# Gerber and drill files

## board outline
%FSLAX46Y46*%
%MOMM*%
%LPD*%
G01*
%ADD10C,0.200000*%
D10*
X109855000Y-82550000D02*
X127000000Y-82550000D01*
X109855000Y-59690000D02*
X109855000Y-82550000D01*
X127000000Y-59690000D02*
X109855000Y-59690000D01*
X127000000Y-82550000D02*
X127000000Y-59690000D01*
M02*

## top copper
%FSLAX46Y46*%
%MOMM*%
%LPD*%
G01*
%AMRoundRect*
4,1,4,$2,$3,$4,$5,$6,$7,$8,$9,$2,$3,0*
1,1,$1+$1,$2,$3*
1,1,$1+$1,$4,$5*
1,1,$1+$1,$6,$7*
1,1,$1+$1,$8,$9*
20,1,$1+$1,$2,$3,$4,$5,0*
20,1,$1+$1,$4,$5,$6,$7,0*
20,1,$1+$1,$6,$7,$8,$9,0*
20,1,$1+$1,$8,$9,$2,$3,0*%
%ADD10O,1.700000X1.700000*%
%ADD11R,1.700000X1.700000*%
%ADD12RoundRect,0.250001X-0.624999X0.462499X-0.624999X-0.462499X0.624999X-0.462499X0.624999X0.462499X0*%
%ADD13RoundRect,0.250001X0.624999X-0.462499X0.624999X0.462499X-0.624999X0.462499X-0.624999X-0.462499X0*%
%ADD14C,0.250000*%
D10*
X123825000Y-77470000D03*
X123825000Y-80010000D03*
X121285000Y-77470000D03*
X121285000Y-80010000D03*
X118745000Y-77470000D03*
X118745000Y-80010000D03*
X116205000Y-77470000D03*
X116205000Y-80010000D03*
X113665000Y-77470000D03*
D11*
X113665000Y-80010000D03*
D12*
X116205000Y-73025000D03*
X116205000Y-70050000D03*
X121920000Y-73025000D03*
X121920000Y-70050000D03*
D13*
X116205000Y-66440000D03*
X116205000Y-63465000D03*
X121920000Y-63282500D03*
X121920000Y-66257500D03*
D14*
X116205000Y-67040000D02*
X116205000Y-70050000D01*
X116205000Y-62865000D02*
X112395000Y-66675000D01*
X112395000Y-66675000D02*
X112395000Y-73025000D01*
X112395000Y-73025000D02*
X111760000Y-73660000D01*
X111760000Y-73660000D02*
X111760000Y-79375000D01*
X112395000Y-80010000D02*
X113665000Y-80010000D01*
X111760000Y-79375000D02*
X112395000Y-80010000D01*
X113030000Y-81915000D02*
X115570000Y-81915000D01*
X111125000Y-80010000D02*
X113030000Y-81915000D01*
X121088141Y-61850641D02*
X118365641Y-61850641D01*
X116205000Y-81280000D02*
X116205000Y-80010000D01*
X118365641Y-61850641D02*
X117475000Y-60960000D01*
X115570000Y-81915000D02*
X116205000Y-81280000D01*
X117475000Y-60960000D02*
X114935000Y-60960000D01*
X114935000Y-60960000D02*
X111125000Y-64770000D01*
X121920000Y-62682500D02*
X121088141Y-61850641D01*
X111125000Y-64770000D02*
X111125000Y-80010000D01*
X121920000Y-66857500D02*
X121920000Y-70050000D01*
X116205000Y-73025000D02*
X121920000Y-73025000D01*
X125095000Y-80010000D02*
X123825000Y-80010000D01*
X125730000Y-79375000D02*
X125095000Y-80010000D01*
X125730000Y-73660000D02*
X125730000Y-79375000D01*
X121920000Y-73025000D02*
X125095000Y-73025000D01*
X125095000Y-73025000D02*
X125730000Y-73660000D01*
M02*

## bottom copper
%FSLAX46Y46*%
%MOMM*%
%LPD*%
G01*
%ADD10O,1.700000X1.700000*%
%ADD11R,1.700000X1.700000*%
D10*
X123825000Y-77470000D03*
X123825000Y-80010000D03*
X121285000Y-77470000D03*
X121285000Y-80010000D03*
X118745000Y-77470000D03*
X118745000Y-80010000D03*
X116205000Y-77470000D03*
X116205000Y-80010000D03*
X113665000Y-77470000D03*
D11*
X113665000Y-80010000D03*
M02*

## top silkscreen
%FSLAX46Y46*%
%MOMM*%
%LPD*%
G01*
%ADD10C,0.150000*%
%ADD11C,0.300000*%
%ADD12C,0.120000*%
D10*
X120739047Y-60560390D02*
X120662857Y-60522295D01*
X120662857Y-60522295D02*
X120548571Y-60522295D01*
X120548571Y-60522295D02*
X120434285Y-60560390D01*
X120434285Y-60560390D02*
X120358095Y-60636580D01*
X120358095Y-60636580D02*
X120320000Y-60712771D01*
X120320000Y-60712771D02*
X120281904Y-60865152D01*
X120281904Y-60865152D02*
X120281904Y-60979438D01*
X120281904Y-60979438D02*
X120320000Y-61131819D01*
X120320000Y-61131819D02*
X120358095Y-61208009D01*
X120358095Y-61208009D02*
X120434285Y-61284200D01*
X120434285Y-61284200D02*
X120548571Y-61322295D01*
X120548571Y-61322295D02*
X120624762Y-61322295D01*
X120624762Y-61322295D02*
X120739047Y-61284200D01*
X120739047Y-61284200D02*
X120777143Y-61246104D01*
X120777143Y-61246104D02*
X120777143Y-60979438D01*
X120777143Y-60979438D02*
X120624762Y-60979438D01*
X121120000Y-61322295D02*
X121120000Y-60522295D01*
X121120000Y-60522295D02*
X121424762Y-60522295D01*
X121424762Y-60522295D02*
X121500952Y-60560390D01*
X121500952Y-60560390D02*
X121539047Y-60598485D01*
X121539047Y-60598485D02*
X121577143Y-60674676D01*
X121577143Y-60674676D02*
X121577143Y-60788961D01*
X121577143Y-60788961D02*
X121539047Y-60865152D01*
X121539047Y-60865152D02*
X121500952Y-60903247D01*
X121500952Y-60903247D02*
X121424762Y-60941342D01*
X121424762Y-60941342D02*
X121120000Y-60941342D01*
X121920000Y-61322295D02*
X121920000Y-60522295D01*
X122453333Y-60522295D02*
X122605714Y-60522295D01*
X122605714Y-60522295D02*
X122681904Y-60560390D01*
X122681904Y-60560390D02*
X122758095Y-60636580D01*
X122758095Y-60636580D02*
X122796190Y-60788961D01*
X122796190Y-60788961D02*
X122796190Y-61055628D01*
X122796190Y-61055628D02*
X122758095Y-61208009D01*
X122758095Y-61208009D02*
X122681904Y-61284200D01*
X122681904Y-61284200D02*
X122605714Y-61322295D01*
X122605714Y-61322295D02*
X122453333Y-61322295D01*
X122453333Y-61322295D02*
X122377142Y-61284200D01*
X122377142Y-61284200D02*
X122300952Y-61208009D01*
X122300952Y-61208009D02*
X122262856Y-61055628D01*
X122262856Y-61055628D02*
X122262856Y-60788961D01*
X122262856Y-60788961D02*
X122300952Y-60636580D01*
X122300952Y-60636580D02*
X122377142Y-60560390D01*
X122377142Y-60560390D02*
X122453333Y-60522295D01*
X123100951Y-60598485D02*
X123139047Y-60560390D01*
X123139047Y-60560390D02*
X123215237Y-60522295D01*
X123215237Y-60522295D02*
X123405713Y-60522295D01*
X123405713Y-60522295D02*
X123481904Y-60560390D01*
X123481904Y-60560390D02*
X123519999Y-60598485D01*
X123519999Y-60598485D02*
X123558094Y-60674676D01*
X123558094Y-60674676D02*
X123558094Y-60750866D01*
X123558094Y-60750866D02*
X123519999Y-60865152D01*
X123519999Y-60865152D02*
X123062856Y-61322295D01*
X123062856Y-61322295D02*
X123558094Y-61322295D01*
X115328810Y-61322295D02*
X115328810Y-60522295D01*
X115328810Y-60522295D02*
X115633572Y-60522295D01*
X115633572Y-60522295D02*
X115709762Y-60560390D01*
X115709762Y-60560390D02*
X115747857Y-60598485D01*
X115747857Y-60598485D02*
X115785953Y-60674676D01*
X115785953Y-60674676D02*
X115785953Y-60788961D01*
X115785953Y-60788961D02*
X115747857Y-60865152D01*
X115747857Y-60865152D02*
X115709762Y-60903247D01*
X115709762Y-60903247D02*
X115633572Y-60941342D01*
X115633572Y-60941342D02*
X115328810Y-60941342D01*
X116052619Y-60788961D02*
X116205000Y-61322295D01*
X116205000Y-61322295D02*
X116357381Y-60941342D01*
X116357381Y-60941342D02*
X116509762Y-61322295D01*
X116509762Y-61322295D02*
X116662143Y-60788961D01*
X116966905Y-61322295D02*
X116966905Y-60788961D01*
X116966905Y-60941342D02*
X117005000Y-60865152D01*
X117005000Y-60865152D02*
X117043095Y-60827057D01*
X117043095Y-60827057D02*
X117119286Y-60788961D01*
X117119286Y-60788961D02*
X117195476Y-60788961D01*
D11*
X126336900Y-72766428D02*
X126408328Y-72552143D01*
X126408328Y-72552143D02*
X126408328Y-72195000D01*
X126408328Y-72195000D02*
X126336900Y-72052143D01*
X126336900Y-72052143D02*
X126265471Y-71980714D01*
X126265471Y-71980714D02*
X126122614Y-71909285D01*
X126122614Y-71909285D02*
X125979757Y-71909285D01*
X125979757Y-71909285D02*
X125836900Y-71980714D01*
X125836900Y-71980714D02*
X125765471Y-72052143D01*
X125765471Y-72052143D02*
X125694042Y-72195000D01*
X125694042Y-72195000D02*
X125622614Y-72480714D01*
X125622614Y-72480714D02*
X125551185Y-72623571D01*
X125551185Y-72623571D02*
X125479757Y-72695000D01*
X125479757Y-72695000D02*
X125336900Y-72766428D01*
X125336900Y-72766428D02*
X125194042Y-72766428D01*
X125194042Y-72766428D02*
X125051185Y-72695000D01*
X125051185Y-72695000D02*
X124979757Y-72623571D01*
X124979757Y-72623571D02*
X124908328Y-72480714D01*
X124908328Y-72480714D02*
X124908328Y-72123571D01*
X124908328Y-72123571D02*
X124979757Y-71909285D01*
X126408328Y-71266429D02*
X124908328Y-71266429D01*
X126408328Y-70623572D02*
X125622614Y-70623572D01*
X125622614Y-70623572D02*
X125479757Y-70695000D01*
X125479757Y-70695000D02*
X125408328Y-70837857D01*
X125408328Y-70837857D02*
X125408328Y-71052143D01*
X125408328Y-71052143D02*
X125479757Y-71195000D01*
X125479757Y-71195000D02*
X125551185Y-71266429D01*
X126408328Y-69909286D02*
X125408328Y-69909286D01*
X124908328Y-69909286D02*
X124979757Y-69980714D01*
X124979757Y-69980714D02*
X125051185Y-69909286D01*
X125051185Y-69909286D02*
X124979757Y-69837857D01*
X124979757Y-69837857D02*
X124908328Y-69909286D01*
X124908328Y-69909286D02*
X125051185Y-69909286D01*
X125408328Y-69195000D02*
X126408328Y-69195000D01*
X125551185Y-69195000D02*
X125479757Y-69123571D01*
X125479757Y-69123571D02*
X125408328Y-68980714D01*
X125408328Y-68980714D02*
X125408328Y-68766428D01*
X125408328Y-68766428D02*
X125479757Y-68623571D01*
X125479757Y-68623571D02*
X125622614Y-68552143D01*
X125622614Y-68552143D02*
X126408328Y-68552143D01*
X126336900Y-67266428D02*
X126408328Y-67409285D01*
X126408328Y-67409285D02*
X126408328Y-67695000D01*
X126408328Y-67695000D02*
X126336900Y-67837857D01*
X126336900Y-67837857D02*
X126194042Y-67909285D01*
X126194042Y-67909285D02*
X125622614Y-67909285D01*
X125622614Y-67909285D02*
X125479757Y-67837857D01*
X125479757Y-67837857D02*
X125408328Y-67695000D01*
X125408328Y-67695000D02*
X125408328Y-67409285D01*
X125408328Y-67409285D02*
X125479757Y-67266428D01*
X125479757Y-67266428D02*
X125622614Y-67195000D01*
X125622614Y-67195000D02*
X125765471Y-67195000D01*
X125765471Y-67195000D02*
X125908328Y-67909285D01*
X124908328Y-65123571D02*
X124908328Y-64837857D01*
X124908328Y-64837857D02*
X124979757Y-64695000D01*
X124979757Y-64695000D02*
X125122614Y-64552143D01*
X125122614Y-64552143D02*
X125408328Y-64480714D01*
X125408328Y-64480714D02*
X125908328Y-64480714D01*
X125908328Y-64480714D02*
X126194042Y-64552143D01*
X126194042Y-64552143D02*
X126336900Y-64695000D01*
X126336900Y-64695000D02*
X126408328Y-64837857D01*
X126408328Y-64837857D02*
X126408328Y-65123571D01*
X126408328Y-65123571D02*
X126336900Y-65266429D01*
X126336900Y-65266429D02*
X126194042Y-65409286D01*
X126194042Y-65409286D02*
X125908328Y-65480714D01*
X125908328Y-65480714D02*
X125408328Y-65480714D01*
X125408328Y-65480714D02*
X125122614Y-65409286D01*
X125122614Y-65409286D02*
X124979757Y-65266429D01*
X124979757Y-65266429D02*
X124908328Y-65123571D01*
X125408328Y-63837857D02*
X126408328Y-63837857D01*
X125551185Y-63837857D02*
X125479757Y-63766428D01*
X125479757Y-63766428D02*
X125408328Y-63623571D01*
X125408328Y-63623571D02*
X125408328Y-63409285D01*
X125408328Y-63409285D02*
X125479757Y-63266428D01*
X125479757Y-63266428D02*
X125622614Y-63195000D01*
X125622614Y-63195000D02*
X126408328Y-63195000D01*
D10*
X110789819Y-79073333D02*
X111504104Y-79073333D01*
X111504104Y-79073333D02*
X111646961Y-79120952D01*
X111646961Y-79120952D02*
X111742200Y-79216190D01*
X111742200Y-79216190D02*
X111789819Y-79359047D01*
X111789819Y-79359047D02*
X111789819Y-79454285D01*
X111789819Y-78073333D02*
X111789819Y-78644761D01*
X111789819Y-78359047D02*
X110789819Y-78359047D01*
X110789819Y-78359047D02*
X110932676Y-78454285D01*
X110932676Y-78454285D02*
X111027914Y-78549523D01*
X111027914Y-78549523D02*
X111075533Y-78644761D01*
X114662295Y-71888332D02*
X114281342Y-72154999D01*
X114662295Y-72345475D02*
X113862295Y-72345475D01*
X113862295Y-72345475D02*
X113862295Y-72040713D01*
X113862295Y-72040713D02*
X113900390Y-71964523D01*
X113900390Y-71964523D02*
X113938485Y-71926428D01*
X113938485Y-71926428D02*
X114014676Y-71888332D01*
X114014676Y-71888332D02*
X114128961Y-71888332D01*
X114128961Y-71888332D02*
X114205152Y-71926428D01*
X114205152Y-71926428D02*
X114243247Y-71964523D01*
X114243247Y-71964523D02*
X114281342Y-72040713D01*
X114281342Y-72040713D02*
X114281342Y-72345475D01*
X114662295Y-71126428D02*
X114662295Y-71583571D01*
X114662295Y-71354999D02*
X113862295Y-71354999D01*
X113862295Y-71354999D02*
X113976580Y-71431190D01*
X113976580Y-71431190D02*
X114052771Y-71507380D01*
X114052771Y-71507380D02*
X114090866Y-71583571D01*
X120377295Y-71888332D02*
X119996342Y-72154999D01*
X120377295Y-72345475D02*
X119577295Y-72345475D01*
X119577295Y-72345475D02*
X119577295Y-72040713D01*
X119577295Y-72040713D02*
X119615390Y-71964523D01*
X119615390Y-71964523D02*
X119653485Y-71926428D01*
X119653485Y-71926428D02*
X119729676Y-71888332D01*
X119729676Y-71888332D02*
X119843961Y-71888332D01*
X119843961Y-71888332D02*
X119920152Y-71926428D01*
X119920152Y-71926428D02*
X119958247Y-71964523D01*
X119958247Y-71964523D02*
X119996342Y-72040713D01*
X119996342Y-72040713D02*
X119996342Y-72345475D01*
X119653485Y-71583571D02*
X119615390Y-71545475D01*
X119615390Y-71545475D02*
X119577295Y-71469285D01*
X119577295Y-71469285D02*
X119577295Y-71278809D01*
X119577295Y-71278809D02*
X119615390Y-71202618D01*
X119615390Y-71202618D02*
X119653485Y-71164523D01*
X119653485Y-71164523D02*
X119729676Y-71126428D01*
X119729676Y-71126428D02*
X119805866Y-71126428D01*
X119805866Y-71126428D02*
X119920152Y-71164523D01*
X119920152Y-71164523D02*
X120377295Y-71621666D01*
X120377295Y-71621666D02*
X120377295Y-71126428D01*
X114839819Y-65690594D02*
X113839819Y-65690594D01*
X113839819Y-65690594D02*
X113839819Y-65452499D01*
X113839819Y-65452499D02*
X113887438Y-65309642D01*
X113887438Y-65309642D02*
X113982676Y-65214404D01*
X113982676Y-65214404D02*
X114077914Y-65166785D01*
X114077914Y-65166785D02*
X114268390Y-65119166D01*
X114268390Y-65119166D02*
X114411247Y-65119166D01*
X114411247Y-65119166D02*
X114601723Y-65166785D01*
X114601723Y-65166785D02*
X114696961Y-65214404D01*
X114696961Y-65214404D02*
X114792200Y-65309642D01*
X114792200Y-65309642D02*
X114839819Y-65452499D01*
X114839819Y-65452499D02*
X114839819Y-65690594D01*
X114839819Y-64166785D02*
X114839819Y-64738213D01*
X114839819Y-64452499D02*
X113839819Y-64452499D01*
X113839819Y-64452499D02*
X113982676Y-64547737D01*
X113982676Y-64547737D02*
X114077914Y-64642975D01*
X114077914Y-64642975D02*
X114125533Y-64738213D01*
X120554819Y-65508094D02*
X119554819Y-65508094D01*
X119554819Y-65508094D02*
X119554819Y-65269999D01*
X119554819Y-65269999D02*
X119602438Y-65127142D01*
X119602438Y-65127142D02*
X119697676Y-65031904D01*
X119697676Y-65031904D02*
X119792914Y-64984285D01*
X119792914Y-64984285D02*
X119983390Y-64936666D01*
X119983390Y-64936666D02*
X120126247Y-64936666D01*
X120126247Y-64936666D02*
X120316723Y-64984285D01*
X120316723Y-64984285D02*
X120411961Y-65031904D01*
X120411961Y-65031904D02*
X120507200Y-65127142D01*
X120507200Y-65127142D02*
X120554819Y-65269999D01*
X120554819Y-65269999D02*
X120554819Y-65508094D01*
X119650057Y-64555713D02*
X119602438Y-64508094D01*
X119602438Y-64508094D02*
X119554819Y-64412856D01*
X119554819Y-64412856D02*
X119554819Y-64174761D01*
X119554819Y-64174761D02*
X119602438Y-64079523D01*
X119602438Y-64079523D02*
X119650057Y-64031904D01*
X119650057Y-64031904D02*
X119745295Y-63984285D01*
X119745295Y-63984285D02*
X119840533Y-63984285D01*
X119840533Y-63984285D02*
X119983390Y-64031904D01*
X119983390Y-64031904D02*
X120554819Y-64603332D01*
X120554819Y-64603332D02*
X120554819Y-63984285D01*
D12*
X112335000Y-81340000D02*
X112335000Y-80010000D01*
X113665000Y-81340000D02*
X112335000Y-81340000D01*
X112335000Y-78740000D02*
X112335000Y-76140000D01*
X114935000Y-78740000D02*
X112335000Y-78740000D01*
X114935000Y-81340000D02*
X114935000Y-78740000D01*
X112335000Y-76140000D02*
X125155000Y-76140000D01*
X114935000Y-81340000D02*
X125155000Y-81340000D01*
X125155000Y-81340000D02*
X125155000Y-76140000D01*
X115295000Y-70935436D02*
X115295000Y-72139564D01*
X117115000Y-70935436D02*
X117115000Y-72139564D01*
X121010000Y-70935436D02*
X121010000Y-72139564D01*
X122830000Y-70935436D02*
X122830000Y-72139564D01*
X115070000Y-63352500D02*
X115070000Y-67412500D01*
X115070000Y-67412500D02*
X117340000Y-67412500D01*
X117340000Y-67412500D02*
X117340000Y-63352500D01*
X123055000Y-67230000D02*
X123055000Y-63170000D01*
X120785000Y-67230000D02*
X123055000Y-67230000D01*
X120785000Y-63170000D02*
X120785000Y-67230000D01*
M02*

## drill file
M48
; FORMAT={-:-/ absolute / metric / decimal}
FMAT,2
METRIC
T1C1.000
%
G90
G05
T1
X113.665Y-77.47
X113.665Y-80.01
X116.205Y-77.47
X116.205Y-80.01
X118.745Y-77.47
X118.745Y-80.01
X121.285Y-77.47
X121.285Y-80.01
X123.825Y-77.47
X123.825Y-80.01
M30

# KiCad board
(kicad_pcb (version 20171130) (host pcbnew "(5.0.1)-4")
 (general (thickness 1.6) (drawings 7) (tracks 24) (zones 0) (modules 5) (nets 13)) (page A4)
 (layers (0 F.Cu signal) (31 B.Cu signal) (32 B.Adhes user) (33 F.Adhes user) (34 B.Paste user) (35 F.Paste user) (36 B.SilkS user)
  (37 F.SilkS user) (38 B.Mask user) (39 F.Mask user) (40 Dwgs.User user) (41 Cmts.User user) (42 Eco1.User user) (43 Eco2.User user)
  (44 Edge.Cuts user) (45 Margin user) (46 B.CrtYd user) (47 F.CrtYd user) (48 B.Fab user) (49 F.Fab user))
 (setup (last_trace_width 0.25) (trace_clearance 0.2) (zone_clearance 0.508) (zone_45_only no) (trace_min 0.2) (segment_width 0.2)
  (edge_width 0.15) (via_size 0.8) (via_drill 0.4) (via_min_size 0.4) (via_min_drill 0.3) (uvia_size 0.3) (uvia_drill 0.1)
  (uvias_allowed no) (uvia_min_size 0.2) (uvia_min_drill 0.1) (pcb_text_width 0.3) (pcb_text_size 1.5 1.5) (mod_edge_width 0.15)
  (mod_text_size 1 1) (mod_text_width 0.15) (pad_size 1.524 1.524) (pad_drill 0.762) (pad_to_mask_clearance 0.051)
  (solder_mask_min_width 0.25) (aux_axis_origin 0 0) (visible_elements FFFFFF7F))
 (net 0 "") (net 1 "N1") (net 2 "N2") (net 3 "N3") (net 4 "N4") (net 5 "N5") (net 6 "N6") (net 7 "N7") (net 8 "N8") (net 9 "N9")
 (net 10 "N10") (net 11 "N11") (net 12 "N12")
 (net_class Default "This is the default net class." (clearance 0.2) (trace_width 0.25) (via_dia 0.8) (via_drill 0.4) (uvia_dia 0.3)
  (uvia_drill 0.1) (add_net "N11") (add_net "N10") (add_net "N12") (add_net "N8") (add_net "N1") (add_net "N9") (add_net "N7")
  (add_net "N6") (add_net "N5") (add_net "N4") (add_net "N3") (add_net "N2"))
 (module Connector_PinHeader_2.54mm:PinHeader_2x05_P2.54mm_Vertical (layer F.Cu) (at 113.665 80.01 90)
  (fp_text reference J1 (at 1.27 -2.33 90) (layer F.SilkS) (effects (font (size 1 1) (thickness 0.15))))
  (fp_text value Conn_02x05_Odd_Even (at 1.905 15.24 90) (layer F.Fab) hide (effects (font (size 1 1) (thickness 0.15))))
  (fp_line (start -1.33 -1.33) (end 0 -1.33) (layer F.SilkS) (width 0.12))
  (fp_line (start -1.33 0) (end -1.33 -1.33) (layer F.SilkS) (width 0.12))
  (fp_line (start 1.27 -1.33) (end 3.87 -1.33) (layer F.SilkS) (width 0.12))
  (fp_line (start 1.27 1.27) (end 1.27 -1.33) (layer F.SilkS) (width 0.12))
  (fp_line (start -1.33 1.27) (end 1.27 1.27) (layer F.SilkS) (width 0.12))
  (fp_line (start 3.87 -1.33) (end 3.87 11.49) (layer F.SilkS) (width 0.12))
  (fp_line (start -1.33 1.27) (end -1.33 11.49) (layer F.SilkS) (width 0.12))
  (fp_line (start -1.33 11.49) (end 3.87 11.49) (layer F.SilkS) (width 0.12))
  (pad 10 thru_hole oval (at 2.54 10.16 90) (size 1.7 1.7) (drill 1) (layers *.Cu *.Mask) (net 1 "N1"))
  (pad 9 thru_hole oval (at 0 10.16 90) (size 1.7 1.7) (drill 1) (layers *.Cu *.Mask) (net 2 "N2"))
  (pad 8 thru_hole oval (at 2.54 7.62 90) (size 1.7 1.7) (drill 1) (layers *.Cu *.Mask) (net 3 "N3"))
  (pad 7 thru_hole oval (at 0 7.62 90) (size 1.7 1.7) (drill 1) (layers *.Cu *.Mask) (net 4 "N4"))
  (pad 6 thru_hole oval (at 2.54 5.08 90) (size 1.7 1.7) (drill 1) (layers *.Cu *.Mask) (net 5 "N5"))
  (pad 5 thru_hole oval (at 0 5.08 90) (size 1.7 1.7) (drill 1) (layers *.Cu *.Mask) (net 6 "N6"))
  (pad 4 thru_hole oval (at 2.54 2.54 90) (size 1.7 1.7) (drill 1) (layers *.Cu *.Mask) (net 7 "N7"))
  (pad 3 thru_hole oval (at 0 2.54 90) (size 1.7 1.7) (drill 1) (layers *.Cu *.Mask) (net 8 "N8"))
  (pad 2 thru_hole oval (at 2.54 0 90) (size 1.7 1.7) (drill 1) (layers *.Cu *.Mask) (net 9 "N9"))
  (pad 1 thru_hole rect (at 0 0 90) (size 1.7 1.7) (drill 1) (layers *.Cu *.Mask) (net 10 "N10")))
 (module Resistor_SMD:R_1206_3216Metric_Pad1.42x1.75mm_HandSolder (layer F.Cu) (at 116.205 71.5375 270)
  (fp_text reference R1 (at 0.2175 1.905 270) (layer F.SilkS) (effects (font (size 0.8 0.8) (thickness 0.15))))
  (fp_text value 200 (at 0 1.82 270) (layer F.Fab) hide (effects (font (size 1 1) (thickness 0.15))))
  (fp_line (start -0.602064 0.91) (end 0.602064 0.91) (layer F.SilkS) (width 0.12))
  (fp_line (start -0.602064 -0.91) (end 0.602064 -0.91) (layer F.SilkS) (width 0.12))
  (pad 2 smd roundrect (at 1.4875 0 270) (size 1.425 1.75) (layers F.Cu F.Paste F.Mask) (roundrect_rratio 0.175439) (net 2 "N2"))
  (pad 1 smd roundrect (at -1.4875 0 270) (size 1.425 1.75) (layers F.Cu F.Paste F.Mask) (roundrect_rratio 0.175439) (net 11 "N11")))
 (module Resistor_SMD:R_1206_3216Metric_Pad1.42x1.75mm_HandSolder (layer F.Cu) (at 121.92 71.5375 270)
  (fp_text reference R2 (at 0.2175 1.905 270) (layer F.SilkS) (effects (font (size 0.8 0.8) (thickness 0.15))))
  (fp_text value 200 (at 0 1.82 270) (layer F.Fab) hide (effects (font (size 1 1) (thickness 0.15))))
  (fp_line (start -0.602064 0.91) (end 0.602064 0.91) (layer F.SilkS) (width 0.12))
  (fp_line (start -0.602064 -0.91) (end 0.602064 -0.91) (layer F.SilkS) (width 0.12))
  (pad 2 smd roundrect (at 1.4875 0 270) (size 1.425 1.75) (layers F.Cu F.Paste F.Mask) (roundrect_rratio 0.175439) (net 2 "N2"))
  (pad 1 smd roundrect (at -1.4875 0 270) (size 1.425 1.75) (layers F.Cu F.Paste F.Mask) (roundrect_rratio 0.175439) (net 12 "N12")))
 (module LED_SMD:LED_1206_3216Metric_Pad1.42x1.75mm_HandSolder (layer F.Cu) (at 116.205 64.9525 90)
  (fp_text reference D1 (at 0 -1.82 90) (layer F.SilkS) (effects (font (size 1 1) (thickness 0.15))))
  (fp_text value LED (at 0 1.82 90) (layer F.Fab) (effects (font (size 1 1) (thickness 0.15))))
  (fp_line (start 1.6 -1.135) (end -2.46 -1.135) (layer F.SilkS) (width 0.12))
  (fp_line (start -2.46 -1.135) (end -2.46 1.135) (layer F.SilkS) (width 0.12))
  (fp_line (start -2.46 1.135) (end 1.6 1.135) (layer F.SilkS) (width 0.12))
  (pad 1 smd roundrect (at -1.4875 0 90) (size 1.425 1.75) (layers F.Cu F.Paste F.Mask) (roundrect_rratio 0.175439) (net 11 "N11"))
  (pad 2 smd roundrect (at 1.4875 0 90) (size 1.425 1.75) (layers F.Cu F.Paste F.Mask) (roundrect_rratio 0.175439) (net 10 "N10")))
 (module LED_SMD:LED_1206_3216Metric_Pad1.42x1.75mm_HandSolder (layer F.Cu) (at 121.92 64.77 90)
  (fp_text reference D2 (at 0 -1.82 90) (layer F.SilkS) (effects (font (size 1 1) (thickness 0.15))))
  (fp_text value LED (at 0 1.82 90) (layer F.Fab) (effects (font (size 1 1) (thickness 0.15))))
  (fp_line (start -2.46 1.135) (end 1.6 1.135) (layer F.SilkS) (width 0.12))
  (fp_line (start -2.46 -1.135) (end -2.46 1.135) (layer F.SilkS) (width 0.12))
  (fp_line (start 1.6 -1.135) (end -2.46 -1.135) (layer F.SilkS) (width 0.12))
  (pad 2 smd roundrect (at 1.4875 0 90) (size 1.425 1.75) (layers F.Cu F.Paste F.Mask) (roundrect_rratio 0.175439) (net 8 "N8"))
  (pad 1 smd roundrect (at -1.4875 0 90) (size 1.425 1.75) (layers F.Cu F.Paste F.Mask) (roundrect_rratio 0.175439) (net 12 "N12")))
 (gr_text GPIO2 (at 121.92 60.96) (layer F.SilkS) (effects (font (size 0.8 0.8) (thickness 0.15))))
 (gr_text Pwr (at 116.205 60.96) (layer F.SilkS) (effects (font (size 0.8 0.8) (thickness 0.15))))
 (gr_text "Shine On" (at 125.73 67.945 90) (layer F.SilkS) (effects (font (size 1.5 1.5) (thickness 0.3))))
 (gr_line (start 109.855 82.55) (end 127 82.55) (layer Edge.Cuts) (width 0.2))
 (gr_line (start 109.855 59.69) (end 109.855 82.55) (layer Edge.Cuts) (width 0.2))
 (gr_line (start 127 59.69) (end 109.855 59.69) (layer Edge.Cuts) (width 0.2))
 (gr_line (start 127 82.55) (end 127 59.69) (layer Edge.Cuts) (width 0.2))
 (segment (start 116.205 67.04) (end 116.205 70.05) (width 0.25) (layer F.Cu) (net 11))
 (segment (start 116.205 62.865) (end 112.395 66.675) (width 0.25) (layer F.Cu) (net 10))
 (segment (start 112.395 66.675) (end 112.395 73.025) (width 0.25) (layer F.Cu) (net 10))
 (segment (start 112.395 73.025) (end 111.76 73.66) (width 0.25) (layer F.Cu) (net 10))
 (segment (start 111.76 73.66) (end 111.76 79.375) (width 0.25) (layer F.Cu) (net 10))
 (segment (start 112.395 80.01) (end 113.665 80.01) (width 0.25) (layer F.Cu) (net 10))
 (segment (start 111.76 79.375) (end 112.395 80.01) (width 0.25) (layer F.Cu) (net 10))
 (segment (start 113.03 81.915) (end 115.57 81.915) (width 0.25) (layer F.Cu) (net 8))
 (segment (start 111.125 80.01) (end 113.03 81.915) (width 0.25) (layer F.Cu) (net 8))
 (segment (start 121.088141 61.850641) (end 118.365641 61.850641) (width 0.25) (layer F.Cu) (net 8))
 (segment (start 116.205 81.28) (end 116.205 80.01) (width 0.25) (layer F.Cu) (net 8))
 (segment (start 118.365641 61.850641) (end 117.475 60.96) (width 0.25) (layer F.Cu) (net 8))
 (segment (start 115.57 81.915) (end 116.205 81.28) (width 0.25) (layer F.Cu) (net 8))
 (segment (start 117.475 60.96) (end 114.935 60.96) (width 0.25) (layer F.Cu) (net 8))
 (segment (start 114.935 60.96) (end 111.125 64.77) (width 0.25) (layer F.Cu) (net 8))
 (segment (start 121.92 62.6825) (end 121.088141 61.850641) (width 0.25) (layer F.Cu) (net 8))
 (segment (start 111.125 64.77) (end 111.125 80.01) (width 0.25) (layer F.Cu) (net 8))
 (segment (start 121.92 66.8575) (end 121.92 70.05) (width 0.25) (layer F.Cu) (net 12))
 (segment (start 116.205 73.025) (end 121.92 73.025) (width 0.25) (layer F.Cu) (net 2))
 (segment (start 125.095 80.01) (end 123.825 80.01) (width 0.25) (layer F.Cu) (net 2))
 (segment (start 125.73 79.375) (end 125.095 80.01) (width 0.25) (layer F.Cu) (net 2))
 (segment (start 125.73 73.66) (end 125.73 79.375) (width 0.25) (layer F.Cu) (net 2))
 (segment (start 121.92 73.025) (end 125.095 73.025) (width 0.25) (layer F.Cu) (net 2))
 (segment (start 125.095 73.025) (end 125.73 73.66) (width 0.25) (layer F.Cu) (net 2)))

